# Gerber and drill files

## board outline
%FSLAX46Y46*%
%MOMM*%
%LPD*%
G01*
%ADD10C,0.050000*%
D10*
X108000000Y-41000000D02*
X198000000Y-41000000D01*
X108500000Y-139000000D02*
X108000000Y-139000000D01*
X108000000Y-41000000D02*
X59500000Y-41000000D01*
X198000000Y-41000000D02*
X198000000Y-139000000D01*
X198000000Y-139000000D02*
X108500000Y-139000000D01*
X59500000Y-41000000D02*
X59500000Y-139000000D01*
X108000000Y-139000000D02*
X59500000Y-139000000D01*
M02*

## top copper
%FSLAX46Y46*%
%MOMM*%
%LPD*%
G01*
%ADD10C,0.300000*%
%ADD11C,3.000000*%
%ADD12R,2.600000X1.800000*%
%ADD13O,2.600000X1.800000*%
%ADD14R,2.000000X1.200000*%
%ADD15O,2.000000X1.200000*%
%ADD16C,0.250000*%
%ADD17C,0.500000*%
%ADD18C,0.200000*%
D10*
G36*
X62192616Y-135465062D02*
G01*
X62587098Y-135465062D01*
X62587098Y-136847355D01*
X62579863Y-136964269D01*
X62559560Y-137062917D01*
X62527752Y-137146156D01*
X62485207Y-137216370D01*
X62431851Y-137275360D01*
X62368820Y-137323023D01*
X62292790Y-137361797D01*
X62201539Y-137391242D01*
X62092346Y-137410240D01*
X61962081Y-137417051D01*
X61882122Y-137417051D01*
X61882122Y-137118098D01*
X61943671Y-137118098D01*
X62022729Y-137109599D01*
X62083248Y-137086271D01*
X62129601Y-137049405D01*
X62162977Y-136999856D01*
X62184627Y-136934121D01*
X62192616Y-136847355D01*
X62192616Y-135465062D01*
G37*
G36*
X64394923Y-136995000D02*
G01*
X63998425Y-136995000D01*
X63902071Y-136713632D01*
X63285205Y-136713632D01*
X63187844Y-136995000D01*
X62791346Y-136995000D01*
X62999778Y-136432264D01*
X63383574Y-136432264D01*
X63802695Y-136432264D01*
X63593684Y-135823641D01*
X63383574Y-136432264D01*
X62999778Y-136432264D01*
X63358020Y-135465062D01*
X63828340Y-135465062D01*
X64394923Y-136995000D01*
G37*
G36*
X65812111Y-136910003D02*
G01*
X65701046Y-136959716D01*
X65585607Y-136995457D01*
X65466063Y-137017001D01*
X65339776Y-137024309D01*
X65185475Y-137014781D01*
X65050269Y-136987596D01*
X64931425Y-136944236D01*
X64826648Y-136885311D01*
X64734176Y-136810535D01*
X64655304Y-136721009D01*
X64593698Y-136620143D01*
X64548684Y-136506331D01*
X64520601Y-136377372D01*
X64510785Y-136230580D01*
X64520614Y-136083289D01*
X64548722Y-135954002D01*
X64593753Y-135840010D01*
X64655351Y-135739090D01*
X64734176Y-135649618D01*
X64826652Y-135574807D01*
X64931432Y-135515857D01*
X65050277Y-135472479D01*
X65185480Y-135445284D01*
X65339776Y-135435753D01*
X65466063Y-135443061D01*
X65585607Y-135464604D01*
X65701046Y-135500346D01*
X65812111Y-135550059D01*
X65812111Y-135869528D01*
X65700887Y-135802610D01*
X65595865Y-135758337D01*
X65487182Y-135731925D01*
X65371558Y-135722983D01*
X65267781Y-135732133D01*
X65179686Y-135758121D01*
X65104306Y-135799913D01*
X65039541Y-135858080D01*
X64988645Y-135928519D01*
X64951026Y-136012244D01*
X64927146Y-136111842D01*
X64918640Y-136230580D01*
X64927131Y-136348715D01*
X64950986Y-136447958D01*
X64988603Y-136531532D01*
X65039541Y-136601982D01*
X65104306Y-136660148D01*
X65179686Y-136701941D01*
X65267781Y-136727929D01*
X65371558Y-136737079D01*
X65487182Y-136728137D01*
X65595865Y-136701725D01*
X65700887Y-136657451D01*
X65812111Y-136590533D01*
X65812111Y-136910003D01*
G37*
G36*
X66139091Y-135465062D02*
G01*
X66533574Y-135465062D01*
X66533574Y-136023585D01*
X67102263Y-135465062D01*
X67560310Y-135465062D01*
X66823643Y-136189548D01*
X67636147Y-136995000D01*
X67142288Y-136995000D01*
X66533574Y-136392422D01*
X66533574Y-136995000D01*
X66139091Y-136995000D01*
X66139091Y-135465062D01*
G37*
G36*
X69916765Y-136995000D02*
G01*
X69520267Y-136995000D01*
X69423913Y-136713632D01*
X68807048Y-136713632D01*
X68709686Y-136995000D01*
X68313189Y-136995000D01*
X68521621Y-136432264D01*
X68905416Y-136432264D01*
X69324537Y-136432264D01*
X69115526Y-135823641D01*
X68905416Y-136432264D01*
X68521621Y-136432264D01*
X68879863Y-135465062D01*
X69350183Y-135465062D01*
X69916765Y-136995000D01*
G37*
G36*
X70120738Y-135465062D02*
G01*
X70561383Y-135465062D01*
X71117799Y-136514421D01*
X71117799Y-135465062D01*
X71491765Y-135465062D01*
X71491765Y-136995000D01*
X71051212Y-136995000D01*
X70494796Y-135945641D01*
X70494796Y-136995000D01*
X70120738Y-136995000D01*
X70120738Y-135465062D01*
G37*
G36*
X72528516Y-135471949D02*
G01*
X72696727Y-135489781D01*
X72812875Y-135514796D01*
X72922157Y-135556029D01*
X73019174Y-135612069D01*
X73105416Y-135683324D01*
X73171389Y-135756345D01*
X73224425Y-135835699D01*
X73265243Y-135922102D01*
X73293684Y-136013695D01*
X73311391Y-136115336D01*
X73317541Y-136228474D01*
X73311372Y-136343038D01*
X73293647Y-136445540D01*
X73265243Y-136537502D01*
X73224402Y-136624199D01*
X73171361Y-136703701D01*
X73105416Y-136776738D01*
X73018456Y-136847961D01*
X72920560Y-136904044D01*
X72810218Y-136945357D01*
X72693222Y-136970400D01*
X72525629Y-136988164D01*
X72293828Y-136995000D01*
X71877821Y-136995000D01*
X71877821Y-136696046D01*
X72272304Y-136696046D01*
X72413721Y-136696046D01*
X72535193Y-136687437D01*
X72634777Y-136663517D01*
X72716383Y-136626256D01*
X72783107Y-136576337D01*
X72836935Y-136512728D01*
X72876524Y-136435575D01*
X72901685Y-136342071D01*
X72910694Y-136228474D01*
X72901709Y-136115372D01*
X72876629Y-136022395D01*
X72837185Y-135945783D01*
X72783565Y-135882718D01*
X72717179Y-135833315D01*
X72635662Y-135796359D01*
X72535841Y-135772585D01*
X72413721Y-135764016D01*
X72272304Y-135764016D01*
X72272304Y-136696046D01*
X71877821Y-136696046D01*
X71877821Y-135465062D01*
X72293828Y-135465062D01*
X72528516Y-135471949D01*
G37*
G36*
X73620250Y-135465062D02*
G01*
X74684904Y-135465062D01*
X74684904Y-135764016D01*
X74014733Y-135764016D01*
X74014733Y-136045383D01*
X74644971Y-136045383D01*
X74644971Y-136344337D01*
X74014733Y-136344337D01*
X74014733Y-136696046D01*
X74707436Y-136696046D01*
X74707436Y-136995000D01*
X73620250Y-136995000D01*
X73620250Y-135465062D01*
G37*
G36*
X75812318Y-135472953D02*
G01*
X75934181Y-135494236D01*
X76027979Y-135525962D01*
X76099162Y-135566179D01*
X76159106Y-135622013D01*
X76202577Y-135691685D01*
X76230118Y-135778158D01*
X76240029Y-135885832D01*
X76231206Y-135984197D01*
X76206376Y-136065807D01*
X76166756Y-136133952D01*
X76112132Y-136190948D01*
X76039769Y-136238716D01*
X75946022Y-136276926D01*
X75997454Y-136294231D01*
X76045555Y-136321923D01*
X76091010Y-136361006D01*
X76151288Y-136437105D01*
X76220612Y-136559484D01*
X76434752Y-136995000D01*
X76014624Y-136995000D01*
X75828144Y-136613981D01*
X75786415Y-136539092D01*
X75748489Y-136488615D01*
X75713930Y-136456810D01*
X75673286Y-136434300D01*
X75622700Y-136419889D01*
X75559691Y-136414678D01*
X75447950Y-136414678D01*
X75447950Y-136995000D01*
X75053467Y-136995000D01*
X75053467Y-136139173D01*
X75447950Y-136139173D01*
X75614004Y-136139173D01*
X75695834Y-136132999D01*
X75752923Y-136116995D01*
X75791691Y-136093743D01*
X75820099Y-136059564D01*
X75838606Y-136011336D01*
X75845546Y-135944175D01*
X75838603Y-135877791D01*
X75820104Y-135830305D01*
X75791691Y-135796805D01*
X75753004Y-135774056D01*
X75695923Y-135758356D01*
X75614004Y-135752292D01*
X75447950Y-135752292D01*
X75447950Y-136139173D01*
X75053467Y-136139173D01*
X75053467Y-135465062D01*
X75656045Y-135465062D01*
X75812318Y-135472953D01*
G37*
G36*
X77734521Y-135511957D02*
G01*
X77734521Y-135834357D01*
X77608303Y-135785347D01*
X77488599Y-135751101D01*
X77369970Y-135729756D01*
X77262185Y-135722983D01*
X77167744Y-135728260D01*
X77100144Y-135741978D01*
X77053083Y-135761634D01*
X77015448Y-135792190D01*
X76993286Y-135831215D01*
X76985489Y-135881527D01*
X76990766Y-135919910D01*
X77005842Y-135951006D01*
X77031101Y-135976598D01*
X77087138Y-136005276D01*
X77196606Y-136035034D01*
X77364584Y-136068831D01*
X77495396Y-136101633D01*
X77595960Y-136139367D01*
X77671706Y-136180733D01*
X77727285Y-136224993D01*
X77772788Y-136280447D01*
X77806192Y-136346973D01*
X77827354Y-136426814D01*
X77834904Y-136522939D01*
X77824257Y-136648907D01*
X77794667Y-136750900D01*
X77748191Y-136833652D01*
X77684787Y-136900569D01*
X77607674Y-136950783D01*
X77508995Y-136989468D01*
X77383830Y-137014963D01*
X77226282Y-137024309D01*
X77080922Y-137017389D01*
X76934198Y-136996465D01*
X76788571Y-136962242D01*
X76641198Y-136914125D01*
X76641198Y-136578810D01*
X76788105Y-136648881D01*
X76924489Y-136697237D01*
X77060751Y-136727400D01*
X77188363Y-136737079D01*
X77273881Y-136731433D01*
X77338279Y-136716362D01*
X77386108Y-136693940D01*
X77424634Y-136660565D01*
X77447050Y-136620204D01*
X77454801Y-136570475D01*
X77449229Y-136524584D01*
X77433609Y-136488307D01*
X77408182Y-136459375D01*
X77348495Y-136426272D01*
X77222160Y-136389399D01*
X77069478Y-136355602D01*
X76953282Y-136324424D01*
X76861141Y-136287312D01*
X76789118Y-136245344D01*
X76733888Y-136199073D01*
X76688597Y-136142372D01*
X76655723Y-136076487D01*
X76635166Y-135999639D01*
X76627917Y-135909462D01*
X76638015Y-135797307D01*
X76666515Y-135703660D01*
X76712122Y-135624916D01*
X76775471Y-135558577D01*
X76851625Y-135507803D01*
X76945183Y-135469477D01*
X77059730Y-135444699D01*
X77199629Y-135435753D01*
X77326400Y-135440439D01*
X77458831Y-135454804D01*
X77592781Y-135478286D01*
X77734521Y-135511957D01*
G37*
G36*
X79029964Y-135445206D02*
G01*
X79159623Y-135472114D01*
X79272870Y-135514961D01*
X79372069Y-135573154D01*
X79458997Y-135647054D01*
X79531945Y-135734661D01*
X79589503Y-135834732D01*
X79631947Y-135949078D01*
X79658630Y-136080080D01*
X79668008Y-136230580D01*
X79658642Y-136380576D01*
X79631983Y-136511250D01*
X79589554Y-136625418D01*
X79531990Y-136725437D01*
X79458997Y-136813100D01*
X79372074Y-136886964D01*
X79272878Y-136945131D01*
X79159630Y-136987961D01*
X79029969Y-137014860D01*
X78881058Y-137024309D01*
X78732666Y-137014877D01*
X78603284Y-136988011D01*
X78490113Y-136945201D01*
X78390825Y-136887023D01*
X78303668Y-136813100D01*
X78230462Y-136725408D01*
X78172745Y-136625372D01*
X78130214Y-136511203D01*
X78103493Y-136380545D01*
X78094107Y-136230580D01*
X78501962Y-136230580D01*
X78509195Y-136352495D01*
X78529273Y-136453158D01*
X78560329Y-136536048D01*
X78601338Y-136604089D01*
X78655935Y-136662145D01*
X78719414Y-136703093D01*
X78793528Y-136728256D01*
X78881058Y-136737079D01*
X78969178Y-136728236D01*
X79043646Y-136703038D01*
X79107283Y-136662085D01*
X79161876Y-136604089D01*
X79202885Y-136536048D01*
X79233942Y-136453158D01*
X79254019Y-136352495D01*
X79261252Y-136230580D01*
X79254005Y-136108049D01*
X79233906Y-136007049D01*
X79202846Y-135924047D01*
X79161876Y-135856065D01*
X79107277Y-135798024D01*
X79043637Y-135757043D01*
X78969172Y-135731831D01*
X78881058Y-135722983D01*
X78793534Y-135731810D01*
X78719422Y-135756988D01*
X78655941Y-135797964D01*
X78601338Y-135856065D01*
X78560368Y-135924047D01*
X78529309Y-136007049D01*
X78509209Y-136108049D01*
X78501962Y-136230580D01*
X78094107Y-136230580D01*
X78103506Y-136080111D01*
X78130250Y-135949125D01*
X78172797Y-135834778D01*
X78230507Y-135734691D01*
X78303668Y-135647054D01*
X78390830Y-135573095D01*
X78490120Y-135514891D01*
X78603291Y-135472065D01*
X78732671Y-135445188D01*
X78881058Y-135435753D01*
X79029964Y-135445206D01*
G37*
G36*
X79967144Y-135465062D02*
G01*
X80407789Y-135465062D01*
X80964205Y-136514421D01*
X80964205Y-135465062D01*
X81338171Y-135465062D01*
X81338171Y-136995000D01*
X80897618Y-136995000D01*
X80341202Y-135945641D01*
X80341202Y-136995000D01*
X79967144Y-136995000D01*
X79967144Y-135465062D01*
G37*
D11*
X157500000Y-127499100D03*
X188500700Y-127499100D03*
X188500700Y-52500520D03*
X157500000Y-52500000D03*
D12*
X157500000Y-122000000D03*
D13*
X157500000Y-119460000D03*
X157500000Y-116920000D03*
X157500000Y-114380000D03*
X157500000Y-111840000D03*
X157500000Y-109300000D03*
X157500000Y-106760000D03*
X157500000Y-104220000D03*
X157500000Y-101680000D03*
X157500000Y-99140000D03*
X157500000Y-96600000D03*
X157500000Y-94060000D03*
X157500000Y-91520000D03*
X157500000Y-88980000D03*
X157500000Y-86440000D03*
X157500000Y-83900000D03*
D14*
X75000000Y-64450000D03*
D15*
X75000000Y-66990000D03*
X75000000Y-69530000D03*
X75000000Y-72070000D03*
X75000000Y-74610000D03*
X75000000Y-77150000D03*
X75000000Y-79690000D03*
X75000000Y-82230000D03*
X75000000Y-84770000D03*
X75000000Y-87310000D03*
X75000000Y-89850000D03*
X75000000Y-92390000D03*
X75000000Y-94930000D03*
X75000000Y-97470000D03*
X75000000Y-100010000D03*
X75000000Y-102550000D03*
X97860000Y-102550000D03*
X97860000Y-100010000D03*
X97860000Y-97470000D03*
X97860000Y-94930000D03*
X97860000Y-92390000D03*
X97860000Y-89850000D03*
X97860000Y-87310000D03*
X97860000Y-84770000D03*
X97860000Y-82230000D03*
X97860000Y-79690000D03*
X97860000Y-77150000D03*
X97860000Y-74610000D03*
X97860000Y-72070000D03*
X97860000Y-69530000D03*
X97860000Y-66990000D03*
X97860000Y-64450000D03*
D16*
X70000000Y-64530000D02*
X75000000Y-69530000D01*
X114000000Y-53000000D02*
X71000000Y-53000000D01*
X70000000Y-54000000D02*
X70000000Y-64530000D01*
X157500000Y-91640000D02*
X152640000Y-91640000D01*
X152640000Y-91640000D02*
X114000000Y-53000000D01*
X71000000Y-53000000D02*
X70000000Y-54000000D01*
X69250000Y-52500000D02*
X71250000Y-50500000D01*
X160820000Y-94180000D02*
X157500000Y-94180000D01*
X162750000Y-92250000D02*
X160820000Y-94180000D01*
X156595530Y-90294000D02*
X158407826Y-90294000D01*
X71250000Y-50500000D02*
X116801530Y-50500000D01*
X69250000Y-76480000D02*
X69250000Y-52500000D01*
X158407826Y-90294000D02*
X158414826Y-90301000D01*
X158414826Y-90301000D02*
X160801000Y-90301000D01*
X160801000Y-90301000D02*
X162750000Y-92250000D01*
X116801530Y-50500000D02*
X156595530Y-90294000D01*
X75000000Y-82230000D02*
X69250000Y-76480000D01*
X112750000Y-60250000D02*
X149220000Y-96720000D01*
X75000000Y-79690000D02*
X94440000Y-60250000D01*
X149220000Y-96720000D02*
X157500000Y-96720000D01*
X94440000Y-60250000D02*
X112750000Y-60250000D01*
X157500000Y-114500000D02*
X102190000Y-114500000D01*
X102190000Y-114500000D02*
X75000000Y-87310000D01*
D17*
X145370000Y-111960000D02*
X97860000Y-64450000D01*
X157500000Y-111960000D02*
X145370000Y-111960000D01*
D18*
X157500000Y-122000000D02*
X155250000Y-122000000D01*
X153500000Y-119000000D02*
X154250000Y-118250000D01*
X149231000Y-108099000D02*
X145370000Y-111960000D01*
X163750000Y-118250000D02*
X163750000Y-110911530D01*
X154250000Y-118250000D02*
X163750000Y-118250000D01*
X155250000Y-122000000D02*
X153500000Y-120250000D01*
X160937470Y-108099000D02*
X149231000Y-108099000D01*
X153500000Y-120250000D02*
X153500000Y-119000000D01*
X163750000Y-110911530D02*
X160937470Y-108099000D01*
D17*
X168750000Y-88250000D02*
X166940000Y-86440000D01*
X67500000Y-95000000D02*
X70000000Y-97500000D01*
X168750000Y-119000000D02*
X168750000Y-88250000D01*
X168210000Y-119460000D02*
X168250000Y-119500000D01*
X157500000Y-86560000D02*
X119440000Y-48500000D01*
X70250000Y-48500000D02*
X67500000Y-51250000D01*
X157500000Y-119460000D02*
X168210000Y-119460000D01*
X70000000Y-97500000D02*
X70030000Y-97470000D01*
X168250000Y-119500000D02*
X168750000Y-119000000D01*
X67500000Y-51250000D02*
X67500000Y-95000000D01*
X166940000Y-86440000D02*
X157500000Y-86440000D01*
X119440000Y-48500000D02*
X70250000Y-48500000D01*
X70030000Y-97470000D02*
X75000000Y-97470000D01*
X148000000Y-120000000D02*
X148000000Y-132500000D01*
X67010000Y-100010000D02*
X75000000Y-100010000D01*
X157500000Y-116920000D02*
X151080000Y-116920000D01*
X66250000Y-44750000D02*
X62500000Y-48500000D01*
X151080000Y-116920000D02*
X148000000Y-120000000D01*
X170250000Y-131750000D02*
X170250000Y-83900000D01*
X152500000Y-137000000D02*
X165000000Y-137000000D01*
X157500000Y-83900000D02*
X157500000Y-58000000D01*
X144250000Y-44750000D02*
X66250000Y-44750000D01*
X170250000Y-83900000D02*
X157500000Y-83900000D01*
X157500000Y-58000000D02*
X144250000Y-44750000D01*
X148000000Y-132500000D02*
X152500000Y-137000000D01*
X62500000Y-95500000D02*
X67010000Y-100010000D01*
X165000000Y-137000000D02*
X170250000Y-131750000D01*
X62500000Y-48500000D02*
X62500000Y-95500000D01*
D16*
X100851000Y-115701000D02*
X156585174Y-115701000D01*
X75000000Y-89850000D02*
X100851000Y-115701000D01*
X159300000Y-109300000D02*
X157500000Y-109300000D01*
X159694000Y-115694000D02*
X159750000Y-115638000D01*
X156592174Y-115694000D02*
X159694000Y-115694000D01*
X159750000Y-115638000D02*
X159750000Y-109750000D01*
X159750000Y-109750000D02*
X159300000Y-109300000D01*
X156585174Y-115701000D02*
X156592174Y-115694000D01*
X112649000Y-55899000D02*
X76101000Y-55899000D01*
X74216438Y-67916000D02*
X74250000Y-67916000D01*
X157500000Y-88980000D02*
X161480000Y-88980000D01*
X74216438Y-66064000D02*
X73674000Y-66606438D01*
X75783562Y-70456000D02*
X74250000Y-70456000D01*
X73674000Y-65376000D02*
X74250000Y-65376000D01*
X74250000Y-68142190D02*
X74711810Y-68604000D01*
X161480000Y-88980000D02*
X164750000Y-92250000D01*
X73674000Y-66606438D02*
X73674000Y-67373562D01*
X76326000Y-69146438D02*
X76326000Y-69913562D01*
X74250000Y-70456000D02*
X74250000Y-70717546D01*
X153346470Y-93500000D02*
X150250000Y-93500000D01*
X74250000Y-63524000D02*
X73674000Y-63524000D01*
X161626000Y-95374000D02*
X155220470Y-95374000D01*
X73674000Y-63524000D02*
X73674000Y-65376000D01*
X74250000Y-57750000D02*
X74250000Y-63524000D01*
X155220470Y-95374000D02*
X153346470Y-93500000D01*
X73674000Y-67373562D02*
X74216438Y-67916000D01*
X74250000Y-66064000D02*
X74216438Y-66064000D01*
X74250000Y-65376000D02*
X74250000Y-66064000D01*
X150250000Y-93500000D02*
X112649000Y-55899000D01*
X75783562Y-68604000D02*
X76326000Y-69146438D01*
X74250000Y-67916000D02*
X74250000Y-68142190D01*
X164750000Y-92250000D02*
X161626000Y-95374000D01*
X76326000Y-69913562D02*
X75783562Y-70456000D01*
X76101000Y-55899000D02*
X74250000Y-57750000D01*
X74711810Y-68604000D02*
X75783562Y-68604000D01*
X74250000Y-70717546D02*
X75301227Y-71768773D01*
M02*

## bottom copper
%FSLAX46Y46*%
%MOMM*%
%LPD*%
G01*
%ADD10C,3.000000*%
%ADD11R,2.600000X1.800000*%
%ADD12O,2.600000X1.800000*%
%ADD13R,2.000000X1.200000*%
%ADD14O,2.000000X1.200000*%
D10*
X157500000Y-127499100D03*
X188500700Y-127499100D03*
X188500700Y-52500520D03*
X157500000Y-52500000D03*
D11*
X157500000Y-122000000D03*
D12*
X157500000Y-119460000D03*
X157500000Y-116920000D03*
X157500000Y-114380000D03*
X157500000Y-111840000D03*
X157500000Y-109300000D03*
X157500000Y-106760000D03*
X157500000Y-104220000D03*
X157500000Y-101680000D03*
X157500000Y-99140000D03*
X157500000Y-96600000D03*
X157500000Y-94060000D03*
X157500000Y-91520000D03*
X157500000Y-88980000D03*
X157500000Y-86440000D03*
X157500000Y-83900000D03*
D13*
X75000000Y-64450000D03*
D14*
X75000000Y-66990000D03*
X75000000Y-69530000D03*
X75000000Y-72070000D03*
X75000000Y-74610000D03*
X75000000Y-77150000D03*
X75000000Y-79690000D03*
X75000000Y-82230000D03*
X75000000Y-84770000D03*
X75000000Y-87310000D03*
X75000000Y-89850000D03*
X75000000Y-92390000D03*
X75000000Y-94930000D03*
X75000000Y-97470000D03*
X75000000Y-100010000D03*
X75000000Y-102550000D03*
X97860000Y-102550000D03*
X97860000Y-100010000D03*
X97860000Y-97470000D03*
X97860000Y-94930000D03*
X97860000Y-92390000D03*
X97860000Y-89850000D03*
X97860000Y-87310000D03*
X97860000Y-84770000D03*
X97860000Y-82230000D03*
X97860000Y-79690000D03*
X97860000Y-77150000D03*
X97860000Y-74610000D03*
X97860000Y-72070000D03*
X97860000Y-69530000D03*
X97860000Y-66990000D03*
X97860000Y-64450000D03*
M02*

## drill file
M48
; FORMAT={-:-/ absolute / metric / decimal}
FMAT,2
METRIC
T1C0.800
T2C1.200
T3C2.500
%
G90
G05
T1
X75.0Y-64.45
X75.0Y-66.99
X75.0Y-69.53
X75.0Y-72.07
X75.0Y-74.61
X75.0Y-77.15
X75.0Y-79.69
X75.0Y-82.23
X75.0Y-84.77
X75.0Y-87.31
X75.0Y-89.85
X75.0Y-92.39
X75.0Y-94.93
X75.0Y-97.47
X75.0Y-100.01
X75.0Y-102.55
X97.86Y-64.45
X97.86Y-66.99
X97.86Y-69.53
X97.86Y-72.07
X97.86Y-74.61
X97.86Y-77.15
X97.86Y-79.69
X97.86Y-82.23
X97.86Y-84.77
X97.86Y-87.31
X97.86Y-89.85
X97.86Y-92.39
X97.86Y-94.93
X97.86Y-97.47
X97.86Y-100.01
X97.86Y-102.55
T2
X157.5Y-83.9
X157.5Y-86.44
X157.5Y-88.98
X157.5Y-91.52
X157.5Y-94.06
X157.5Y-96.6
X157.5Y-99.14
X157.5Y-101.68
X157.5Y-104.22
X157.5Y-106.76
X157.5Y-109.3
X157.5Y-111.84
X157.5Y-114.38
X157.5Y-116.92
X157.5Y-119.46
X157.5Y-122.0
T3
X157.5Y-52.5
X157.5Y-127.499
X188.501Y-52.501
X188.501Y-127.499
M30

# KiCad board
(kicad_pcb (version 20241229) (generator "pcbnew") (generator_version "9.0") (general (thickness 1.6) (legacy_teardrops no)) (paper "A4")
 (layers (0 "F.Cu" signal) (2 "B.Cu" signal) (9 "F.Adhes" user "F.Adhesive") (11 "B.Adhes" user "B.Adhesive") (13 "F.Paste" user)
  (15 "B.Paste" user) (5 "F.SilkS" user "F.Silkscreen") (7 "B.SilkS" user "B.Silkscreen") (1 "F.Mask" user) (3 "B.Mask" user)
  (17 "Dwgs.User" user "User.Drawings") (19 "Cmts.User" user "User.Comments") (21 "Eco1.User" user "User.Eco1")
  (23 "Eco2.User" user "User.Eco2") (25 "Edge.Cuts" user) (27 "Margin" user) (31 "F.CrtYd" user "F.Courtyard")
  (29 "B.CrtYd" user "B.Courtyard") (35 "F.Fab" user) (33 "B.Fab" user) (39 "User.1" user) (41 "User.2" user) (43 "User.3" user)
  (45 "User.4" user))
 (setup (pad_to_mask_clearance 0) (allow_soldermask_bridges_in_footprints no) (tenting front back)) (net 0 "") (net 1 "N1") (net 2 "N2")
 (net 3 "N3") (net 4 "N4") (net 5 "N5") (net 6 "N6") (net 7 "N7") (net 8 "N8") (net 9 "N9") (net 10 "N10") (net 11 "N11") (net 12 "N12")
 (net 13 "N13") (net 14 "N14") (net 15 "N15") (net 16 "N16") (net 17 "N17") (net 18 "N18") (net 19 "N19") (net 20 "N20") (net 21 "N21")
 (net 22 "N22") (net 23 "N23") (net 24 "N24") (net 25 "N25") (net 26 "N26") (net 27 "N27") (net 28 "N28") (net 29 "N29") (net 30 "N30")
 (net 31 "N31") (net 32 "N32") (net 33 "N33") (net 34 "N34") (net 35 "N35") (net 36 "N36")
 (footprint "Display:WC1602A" (layer "F.Cu") (at 157.5 122 90)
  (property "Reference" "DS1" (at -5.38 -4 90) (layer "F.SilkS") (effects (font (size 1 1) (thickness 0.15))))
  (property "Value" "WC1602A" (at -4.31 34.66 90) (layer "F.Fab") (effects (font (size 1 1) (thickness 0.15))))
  (pad "" thru_hole circle (at -5.4991 0 90) (size 3 3) (drill 2.5) (layers "*.Cu" "*.Mask") (remove_unused_layers no))
  (pad "" thru_hole circle (at -5.4991 31.0007 90) (size 3 3) (drill 2.5) (layers "*.Cu" "*.Mask") (remove_unused_layers no))
  (pad "" thru_hole circle (at 69.49948 31.0007 90) (size 3 3) (drill 2.5) (layers "*.Cu" "*.Mask") (remove_unused_layers no))
  (pad "" thru_hole circle (at 69.5 0 90) (size 3 3) (drill 2.5) (layers "*.Cu" "*.Mask") (remove_unused_layers no))
  (pad "1" thru_hole rect (at 0 0 90) (size 1.8 2.6) (drill 1.2) (layers "*.Cu" "*.Mask") (remove_unused_layers no) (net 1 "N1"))
  (pad "2" thru_hole oval (at 2.54 0 90) (size 1.8 2.6) (drill 1.2) (layers "*.Cu" "*.Mask") (remove_unused_layers no) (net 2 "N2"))
  (pad "3" thru_hole oval (at 5.08 0 90) (size 1.8 2.6) (drill 1.2) (layers "*.Cu" "*.Mask") (remove_unused_layers no) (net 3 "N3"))
  (pad "4" thru_hole oval (at 7.62 0 90) (size 1.8 2.6) (drill 1.2) (layers "*.Cu" "*.Mask") (remove_unused_layers no) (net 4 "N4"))
  (pad "5" thru_hole oval (at 10.16 0 90) (size 1.8 2.6) (drill 1.2) (layers "*.Cu" "*.Mask") (remove_unused_layers no) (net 1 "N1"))
  (pad "6" thru_hole oval (at 12.7 0 90) (size 1.8 2.6) (drill 1.2) (layers "*.Cu" "*.Mask") (remove_unused_layers no) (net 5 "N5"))
  (pad "7" thru_hole oval (at 15.24 0 90) (size 1.8 2.6) (drill 1.2) (layers "*.Cu" "*.Mask") (remove_unused_layers no) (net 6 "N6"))
  (pad "8" thru_hole oval (at 17.78 0 90) (size 1.8 2.6) (drill 1.2) (layers "*.Cu" "*.Mask") (remove_unused_layers no) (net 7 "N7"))
  (pad "9" thru_hole oval (at 20.32 0 90) (size 1.8 2.6) (drill 1.2) (layers "*.Cu" "*.Mask") (remove_unused_layers no) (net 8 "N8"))
  (pad "10" thru_hole oval (at 22.86 0 90) (size 1.8 2.6) (drill 1.2) (layers "*.Cu" "*.Mask") (remove_unused_layers no) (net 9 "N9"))
  (pad "11" thru_hole oval (at 25.4 0 90) (size 1.8 2.6) (drill 1.2) (layers "*.Cu" "*.Mask") (remove_unused_layers no) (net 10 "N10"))
  (pad "12" thru_hole oval (at 27.94 0 90) (size 1.8 2.6) (drill 1.2) (layers "*.Cu" "*.Mask") (remove_unused_layers no) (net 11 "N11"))
  (pad "13" thru_hole oval (at 30.48 0 90) (size 1.8 2.6) (drill 1.2) (layers "*.Cu" "*.Mask") (remove_unused_layers no) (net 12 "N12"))
  (pad "14" thru_hole oval (at 33.02 0 90) (size 1.8 2.6) (drill 1.2) (layers "*.Cu" "*.Mask") (remove_unused_layers no) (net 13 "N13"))
  (pad "15" thru_hole oval (at 35.56 0 90) (size 1.8 2.6) (drill 1.2) (layers "*.Cu" "*.Mask") (remove_unused_layers no) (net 2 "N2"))
  (pad "16" thru_hole oval (at 38.1 0 90) (size 1.8 2.6) (drill 1.2) (layers "*.Cu" "*.Mask") (remove_unused_layers no) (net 3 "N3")))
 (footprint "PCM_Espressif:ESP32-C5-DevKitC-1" (layer "F.Cu") (at 74.96012 64.45468)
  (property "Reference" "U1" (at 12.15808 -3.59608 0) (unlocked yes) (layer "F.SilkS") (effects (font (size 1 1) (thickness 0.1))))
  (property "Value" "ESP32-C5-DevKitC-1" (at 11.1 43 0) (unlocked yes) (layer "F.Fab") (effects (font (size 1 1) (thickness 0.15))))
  (pad "1" thru_hole rect (at 0.03988 -0.00468 270) (size 1.2 2) (drill 0.8) (layers "*.Cu" "*.Mask") (remove_unused_layers no)
   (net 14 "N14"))
  (pad "2" thru_hole oval (at 0.03988 2.53532 270) (size 1.2 2) (drill 0.8) (layers "*.Cu" "*.Mask") (remove_unused_layers no)
   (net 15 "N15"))
  (pad "3" thru_hole oval (at 0.03988 5.07532 270) (size 1.2 2) (drill 0.8) (layers "*.Cu" "*.Mask") (remove_unused_layers no)
   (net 12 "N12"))
  (pad "4" thru_hole oval (at 0.03988 7.61532 270) (size 1.2 2) (drill 0.8) (layers "*.Cu" "*.Mask") (remove_unused_layers no)
   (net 13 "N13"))
  (pad "5" thru_hole oval (at 0.03988 10.15532 270) (size 1.2 2) (drill 0.8) (layers "*.Cu" "*.Mask") (remove_unused_layers no)
   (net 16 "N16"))
  (pad "6" thru_hole oval (at 0.03988 12.69532 270) (size 1.2 2) (drill 0.8) (layers "*.Cu" "*.Mask") (remove_unused_layers no)
   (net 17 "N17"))
  (pad "7" thru_hole oval (at 0.03988 15.23532 270) (size 1.2 2) (drill 0.8) (layers "*.Cu" "*.Mask") (remove_unused_layers no)
   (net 10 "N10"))
  (pad "8" thru_hole oval (at 0.03988 17.77532 270) (size 1.2 2) (drill 0.8) (layers "*.Cu" "*.Mask") (remove_unused_layers no)
   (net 11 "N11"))
  (pad "9" thru_hole oval (at 0.03988 20.31532 270) (size 1.2 2) (drill 0.8) (layers "*.Cu" "*.Mask") (remove_unused_layers no)
   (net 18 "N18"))
  (pad "10" thru_hole oval (at 0.03988 22.85532 270) (size 1.2 2) (drill 0.8) (layers "*.Cu" "*.Mask") (remove_unused_layers no)
   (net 4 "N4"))
  (pad "11" thru_hole oval (at 0.03988 25.39532 270) (size 1.2 2) (drill 0.8) (layers "*.Cu" "*.Mask") (remove_unused_layers no)
   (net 5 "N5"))
  (pad "12" thru_hole oval (at 0.03988 27.93532 270) (size 1.2 2) (drill 0.8) (layers "*.Cu" "*.Mask") (remove_unused_layers no)
   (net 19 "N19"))
  (pad "13" thru_hole oval (at 0.03988 30.47532 270) (size 1.2 2) (drill 0.8) (layers "*.Cu" "*.Mask") (remove_unused_layers no)
   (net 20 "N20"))
  (pad "14" thru_hole oval (at 0.03988 33.01532 270) (size 1.2 2) (drill 0.8) (layers "*.Cu" "*.Mask") (remove_unused_layers no)
   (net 2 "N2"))
  (pad "15" thru_hole oval (at 0.03988 35.55532 270) (size 1.2 2) (drill 0.8) (layers "*.Cu" "*.Mask") (remove_unused_layers no)
   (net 3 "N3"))
  (pad "16" thru_hole oval (at 0.03988 38.09532 270) (size 1.2 2) (drill 0.8) (layers "*.Cu" "*.Mask") (remove_unused_layers no)
   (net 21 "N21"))
  (pad "17" thru_hole oval (at 22.89988 38.09532 270) (size 1.2 2) (drill 0.8) (layers "*.Cu" "*.Mask") (remove_unused_layers no)
   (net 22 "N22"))
  (pad "18" thru_hole oval (at 22.89988 35.55532 270) (size 1.2 2) (drill 0.8) (layers "*.Cu" "*.Mask") (remove_unused_layers no)
   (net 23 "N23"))
  (pad "19" thru_hole oval (at 22.89988 33.01532 270) (size 1.2 2) (drill 0.8) (layers "*.Cu" "*.Mask") (remove_unused_layers no)
   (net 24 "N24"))
  (pad "20" thru_hole oval (at 22.89988 30.47532 270) (size 1.2 2) (drill 0.8) (layers "*.Cu" "*.Mask") (remove_unused_layers no)
   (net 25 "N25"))
  (pad "21" thru_hole oval (at 22.89988 27.93532 270) (size 1.2 2) (drill 0.8) (layers "*.Cu" "*.Mask") (remove_unused_layers no)
   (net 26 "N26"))
  (pad "22" thru_hole oval (at 22.89988 25.39532 270) (size 1.2 2) (drill 0.8) (layers "*.Cu" "*.Mask") (remove_unused_layers no)
   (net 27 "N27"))
  (pad "23" thru_hole oval (at 22.89988 22.85532 270) (size 1.2 2) (drill 0.8) (layers "*.Cu" "*.Mask") (remove_unused_layers no)
   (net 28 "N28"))
  (pad "24" thru_hole oval (at 22.89988 20.31532 270) (size 1.2 2) (drill 0.8) (layers "*.Cu" "*.Mask") (remove_unused_layers no)
   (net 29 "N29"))
  (pad "25" thru_hole oval (at 22.89988 17.77532 270) (size 1.2 2) (drill 0.8) (layers "*.Cu" "*.Mask") (remove_unused_layers no)
   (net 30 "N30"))
  (pad "26" thru_hole oval (at 22.89988 15.23532 270) (size 1.2 2) (drill 0.8) (layers "*.Cu" "*.Mask") (remove_unused_layers no)
   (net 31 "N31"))
  (pad "27" thru_hole oval (at 22.89988 12.69532 270) (size 1.2 2) (drill 0.8) (layers "*.Cu" "*.Mask") (remove_unused_layers no)
   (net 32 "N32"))
  (pad "28" thru_hole oval (at 22.89988 10.15532 270) (size 1.2 2) (drill 0.8) (layers "*.Cu" "*.Mask") (remove_unused_layers no)
   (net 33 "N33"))
  (pad "29" thru_hole oval (at 22.89988 7.61532 270) (size 1.2 2) (drill 0.8) (layers "*.Cu" "*.Mask") (remove_unused_layers no)
   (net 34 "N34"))
  (pad "30" thru_hole oval (at 22.89988 5.07532 270) (size 1.2 2) (drill 0.8) (layers "*.Cu" "*.Mask") (remove_unused_layers no)
   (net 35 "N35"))
  (pad "31" thru_hole oval (at 22.89988 2.53532 270) (size 1.2 2) (drill 0.8) (layers "*.Cu" "*.Mask") (remove_unused_layers no)
   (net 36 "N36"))
  (pad "32" thru_hole oval (at 22.89988 -0.00468 270) (size 1.2 2) (drill 0.8) (layers "*.Cu" "*.Mask") (remove_unused_layers no)
   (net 1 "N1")))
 (gr_line (start 108 41) (end 198 41) (stroke (width 0.05) (type default)) (layer "Edge.Cuts"))
 (gr_line (start 108.5 139) (end 108 139) (stroke (width 0.05) (type default)) (layer "Edge.Cuts"))
 (gr_line (start 108 41) (end 59.5 41) (stroke (width 0.05) (type default)) (layer "Edge.Cuts"))
 (gr_line (start 198 41) (end 198 139) (stroke (width 0.05) (type default)) (layer "Edge.Cuts"))
 (gr_line (start 198 139) (end 108.5 139) (stroke (width 0.05) (type default)) (layer "Edge.Cuts"))
 (gr_line (start 59.5 41) (end 59.5 139) (stroke (width 0.05) (type default)) (layer "Edge.Cuts"))
 (gr_line (start 108 139) (end 59.5 139) (stroke (width 0.05) (type default)) (layer "Edge.Cuts"))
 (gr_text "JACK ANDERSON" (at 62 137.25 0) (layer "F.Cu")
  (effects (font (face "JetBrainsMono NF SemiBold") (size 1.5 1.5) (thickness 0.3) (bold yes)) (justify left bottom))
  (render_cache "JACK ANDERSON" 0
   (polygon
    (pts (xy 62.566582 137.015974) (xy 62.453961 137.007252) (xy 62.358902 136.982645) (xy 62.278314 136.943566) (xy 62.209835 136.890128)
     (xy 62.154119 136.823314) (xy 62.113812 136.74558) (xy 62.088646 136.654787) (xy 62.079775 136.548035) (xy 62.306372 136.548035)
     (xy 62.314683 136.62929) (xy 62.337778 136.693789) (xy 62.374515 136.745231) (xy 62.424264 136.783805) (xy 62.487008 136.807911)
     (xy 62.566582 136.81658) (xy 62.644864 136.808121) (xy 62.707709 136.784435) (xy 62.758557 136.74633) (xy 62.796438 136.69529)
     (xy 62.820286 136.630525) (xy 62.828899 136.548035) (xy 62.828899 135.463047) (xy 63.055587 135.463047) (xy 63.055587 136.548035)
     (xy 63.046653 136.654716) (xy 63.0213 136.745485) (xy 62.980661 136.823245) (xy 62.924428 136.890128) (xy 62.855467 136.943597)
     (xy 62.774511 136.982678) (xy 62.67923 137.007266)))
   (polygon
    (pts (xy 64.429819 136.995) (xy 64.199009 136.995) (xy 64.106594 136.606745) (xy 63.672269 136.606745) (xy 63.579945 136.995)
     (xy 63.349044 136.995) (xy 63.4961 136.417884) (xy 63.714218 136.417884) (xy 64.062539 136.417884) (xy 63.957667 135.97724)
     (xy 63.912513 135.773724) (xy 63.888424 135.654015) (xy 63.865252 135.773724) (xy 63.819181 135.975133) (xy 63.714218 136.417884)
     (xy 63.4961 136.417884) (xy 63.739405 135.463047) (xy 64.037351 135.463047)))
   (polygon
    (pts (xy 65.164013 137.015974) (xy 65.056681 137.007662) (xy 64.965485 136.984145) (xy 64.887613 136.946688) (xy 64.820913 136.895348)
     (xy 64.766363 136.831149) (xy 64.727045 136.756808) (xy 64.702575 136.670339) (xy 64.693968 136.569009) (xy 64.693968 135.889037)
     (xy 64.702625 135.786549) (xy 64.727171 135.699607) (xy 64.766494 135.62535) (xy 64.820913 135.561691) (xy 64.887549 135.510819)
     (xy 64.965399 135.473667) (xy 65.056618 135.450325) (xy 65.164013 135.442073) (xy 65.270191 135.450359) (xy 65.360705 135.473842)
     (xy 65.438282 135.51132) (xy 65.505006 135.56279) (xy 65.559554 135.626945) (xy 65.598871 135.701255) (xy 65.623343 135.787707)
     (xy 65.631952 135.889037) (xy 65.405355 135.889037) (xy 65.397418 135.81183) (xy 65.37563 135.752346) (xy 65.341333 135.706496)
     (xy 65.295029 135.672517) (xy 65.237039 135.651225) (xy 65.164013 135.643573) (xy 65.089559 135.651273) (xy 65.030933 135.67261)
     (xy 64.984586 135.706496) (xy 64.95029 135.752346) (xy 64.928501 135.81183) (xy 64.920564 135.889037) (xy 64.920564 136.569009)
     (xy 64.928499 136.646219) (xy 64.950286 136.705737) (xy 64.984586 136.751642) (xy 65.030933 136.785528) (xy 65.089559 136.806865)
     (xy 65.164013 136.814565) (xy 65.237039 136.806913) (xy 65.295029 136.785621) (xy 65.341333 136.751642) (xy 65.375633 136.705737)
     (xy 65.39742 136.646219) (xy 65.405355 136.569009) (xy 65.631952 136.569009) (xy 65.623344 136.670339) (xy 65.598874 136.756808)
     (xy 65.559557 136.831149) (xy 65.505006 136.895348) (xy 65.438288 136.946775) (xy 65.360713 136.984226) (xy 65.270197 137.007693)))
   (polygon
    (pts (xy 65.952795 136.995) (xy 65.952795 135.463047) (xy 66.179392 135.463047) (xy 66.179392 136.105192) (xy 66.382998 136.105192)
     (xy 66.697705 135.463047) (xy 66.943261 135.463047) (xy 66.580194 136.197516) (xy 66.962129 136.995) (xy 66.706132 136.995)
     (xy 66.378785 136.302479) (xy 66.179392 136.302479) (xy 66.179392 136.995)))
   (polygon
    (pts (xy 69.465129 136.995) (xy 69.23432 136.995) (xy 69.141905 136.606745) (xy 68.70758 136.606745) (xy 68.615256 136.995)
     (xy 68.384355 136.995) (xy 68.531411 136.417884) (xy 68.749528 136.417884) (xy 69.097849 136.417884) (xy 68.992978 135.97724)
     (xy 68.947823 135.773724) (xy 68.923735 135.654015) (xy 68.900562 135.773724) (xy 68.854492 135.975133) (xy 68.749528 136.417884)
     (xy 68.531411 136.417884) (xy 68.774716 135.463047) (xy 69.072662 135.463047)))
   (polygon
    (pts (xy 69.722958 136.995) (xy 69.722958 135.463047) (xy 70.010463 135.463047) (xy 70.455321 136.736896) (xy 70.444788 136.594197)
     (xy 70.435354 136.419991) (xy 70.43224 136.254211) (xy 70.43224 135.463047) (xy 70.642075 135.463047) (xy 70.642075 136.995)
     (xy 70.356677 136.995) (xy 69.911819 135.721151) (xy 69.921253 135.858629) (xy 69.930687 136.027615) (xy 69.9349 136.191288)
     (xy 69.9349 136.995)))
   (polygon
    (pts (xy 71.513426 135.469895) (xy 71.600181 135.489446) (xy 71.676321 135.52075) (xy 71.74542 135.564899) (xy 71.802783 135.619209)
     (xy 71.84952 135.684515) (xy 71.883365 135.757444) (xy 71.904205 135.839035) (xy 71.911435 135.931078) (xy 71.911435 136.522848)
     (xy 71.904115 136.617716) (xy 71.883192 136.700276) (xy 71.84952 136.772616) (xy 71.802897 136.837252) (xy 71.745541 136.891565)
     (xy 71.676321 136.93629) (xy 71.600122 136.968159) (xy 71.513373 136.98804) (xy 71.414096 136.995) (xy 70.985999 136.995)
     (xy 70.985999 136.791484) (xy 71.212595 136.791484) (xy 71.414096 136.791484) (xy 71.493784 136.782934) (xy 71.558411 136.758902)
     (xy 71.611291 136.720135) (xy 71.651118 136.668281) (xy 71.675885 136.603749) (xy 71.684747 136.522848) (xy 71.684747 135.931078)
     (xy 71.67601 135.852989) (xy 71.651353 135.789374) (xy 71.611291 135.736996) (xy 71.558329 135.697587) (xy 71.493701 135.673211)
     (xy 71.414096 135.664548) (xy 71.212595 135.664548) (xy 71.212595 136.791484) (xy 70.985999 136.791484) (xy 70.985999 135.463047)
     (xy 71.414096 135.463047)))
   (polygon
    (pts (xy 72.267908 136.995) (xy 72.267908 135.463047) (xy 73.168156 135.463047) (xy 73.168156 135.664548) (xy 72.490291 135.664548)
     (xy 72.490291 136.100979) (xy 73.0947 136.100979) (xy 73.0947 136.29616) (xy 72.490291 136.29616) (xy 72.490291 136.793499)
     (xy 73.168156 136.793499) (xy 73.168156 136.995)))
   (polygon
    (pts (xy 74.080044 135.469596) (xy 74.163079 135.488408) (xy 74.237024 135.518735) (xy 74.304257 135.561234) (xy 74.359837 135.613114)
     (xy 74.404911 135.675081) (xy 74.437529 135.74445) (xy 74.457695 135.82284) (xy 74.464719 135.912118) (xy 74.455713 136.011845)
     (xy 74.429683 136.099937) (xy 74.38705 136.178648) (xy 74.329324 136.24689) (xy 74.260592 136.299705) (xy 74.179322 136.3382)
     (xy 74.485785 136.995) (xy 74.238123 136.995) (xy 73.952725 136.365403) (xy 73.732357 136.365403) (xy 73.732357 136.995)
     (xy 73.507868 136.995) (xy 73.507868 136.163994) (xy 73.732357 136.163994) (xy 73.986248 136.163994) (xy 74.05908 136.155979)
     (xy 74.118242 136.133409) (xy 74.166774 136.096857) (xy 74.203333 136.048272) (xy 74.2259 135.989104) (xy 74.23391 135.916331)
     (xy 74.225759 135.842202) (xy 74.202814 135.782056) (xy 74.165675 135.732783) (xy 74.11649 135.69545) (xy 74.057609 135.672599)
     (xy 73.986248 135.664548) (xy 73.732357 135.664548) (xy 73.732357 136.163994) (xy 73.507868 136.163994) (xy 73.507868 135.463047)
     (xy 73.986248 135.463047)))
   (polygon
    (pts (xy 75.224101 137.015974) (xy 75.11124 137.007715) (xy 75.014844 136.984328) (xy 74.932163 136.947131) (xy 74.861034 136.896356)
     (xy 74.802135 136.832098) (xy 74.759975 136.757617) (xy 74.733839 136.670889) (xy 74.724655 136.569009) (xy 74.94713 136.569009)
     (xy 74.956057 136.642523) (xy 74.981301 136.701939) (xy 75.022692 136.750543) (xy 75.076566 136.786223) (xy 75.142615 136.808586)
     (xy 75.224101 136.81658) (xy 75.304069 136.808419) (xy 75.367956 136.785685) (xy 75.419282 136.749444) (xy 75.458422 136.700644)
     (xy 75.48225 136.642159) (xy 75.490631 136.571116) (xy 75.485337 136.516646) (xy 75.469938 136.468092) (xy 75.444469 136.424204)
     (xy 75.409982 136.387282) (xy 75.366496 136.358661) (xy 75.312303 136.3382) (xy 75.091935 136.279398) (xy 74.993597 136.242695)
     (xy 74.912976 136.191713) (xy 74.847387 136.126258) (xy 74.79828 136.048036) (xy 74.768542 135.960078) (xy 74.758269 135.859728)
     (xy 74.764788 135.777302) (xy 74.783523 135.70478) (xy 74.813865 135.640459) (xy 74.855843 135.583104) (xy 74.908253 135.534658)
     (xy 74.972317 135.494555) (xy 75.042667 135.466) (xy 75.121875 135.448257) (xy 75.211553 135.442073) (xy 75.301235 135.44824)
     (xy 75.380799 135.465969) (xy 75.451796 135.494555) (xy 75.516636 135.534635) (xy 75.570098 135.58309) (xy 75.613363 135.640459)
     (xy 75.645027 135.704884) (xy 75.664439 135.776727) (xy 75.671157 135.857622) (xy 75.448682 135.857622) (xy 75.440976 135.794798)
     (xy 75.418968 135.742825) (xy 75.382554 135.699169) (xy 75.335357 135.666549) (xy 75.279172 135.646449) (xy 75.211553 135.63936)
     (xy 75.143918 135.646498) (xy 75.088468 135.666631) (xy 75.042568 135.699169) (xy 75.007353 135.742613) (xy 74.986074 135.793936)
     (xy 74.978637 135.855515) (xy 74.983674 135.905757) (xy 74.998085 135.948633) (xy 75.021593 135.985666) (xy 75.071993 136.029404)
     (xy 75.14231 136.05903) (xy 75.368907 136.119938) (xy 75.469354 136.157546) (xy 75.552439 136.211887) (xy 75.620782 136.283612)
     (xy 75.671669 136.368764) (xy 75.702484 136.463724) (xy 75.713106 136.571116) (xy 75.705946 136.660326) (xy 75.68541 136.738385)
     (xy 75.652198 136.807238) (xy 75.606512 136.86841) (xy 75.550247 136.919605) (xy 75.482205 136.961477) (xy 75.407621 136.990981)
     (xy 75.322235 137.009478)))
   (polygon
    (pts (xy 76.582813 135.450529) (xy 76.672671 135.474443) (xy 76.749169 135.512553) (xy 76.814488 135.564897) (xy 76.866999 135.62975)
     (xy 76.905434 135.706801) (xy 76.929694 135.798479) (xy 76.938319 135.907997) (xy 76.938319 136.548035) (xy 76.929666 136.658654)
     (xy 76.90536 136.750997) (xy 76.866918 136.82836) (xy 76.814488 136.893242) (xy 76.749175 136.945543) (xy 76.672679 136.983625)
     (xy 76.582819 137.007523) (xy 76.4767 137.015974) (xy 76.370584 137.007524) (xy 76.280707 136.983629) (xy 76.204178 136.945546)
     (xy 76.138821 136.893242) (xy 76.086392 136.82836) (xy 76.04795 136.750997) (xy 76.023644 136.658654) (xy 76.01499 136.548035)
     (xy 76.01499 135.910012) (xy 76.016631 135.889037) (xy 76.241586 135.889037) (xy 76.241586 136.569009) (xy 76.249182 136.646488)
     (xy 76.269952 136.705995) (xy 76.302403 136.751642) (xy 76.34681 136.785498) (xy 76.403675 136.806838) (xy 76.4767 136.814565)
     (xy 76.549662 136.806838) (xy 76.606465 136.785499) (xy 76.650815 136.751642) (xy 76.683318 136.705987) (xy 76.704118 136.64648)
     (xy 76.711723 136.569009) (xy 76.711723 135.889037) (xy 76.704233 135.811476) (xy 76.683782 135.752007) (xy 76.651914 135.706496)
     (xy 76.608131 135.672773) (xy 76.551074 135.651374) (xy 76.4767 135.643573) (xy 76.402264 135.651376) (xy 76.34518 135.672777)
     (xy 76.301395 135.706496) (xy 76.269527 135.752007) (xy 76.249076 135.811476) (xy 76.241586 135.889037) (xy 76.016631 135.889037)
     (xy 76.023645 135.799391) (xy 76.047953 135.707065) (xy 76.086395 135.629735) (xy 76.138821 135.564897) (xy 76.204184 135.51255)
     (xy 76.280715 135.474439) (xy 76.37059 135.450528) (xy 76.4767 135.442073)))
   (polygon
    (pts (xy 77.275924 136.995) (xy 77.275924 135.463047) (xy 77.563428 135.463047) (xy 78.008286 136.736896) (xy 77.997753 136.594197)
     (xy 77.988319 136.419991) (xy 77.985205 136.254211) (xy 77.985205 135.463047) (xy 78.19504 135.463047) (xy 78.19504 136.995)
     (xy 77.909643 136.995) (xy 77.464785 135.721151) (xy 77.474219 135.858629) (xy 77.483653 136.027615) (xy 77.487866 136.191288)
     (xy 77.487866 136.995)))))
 (segment (start 70 64.53) (end 75 69.53) (width 0.25) (layer "F.Cu") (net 12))
 (segment (start 114 53) (end 71 53) (width 0.25) (layer "F.Cu") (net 12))
 (segment (start 70 54) (end 70 64.53) (width 0.25) (layer "F.Cu") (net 12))
 (segment (start 157.5 91.64) (end 152.64 91.64) (width 0.25) (layer "F.Cu") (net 12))
 (segment (start 152.64 91.64) (end 114 53) (width 0.25) (layer "F.Cu") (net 12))
 (segment (start 71 53) (end 70 54) (width 0.25) (layer "F.Cu") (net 12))
 (segment (start 69.25 52.5) (end 71.25 50.5) (width 0.25) (layer "F.Cu") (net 11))
 (segment (start 160.82 94.18) (end 157.5 94.18) (width 0.25) (layer "F.Cu") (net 11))
 (segment (start 162.75 92.25) (end 160.82 94.18) (width 0.25) (layer "F.Cu") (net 11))
 (segment (start 156.59553 90.294) (end 158.407826 90.294) (width 0.25) (layer "F.Cu") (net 11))
 (segment (start 71.25 50.5) (end 116.80153 50.5) (width 0.25) (layer "F.Cu") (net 11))
 (segment (start 69.25 76.48) (end 69.25 52.5) (width 0.25) (layer "F.Cu") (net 11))
 (segment (start 158.407826 90.294) (end 158.414826 90.301) (width 0.25) (layer "F.Cu") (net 11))
 (segment (start 158.414826 90.301) (end 160.801 90.301) (width 0.25) (layer "F.Cu") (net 11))
 (segment (start 160.801 90.301) (end 162.75 92.25) (width 0.25) (layer "F.Cu") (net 11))
 (segment (start 116.80153 50.5) (end 156.59553 90.294) (width 0.25) (layer "F.Cu") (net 11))
 (segment (start 75 82.23) (end 69.25 76.48) (width 0.25) (layer "F.Cu") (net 11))
 (segment (start 112.75 60.25) (end 149.22 96.72) (width 0.25) (layer "F.Cu") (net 10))
 (segment (start 75 79.69) (end 94.44 60.25) (width 0.25) (layer "F.Cu") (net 10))
 (segment (start 149.22 96.72) (end 157.5 96.72) (width 0.25) (layer "F.Cu") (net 10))
 (segment (start 94.44 60.25) (end 112.75 60.25) (width 0.25) (layer "F.Cu") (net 10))
 (segment (start 157.5 114.5) (end 102.19 114.5) (width 0.25) (layer "F.Cu") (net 4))
 (segment (start 102.19 114.5) (end 75 87.31) (width 0.25) (layer "F.Cu") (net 4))
 (segment (start 145.37 111.96) (end 97.86 64.45) (width 0.5) (layer "F.Cu") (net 1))
 (segment (start 157.5 111.96) (end 145.37 111.96) (width 0.5) (layer "F.Cu") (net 1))
 (segment (start 157.5 122) (end 155.25 122) (width 0.2) (layer "F.Cu") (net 1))
 (segment (start 153.5 119) (end 154.25 118.25) (width 0.2) (layer "F.Cu") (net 1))
 (segment (start 149.231 108.099) (end 145.37 111.96) (width 0.2) (layer "F.Cu") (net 1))
 (segment (start 163.75 118.25) (end 163.75 110.91153) (width 0.2) (layer "F.Cu") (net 1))
 (segment (start 154.25 118.25) (end 163.75 118.25) (width 0.2) (layer "F.Cu") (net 1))
 (segment (start 155.25 122) (end 153.5 120.25) (width 0.2) (layer "F.Cu") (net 1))
 (segment (start 160.93747 108.099) (end 149.231 108.099) (width 0.2) (layer "F.Cu") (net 1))
 (segment (start 153.5 120.25) (end 153.5 119) (width 0.2) (layer "F.Cu") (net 1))
 (segment (start 163.75 110.91153) (end 160.93747 108.099) (width 0.2) (layer "F.Cu") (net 1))
 (segment (start 168.75 88.25) (end 166.94 86.44) (width 0.5) (layer "F.Cu") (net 2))
 (segment (start 67.5 95) (end 70 97.5) (width 0.5) (layer "F.Cu") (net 2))
 (segment (start 168.75 119) (end 168.75 88.25) (width 0.5) (layer "F.Cu") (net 2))
 (segment (start 168.21 119.46) (end 168.25 119.5) (width 0.5) (layer "F.Cu") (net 2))
 (segment (start 157.5 86.56) (end 119.44 48.5) (width 0.5) (layer "F.Cu") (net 2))
 (segment (start 70.25 48.5) (end 67.5 51.25) (width 0.5) (layer "F.Cu") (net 2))
 (segment (start 157.5 119.46) (end 168.21 119.46) (width 0.5) (layer "F.Cu") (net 2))
 (segment (start 70 97.5) (end 70.03 97.47) (width 0.5) (layer "F.Cu") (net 2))
 (segment (start 168.25 119.5) (end 168.75 119) (width 0.5) (layer "F.Cu") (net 2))
 (segment (start 67.5 51.25) (end 67.5 95) (width 0.5) (layer "F.Cu") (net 2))
 (segment (start 166.94 86.44) (end 157.5 86.44) (width 0.5) (layer "F.Cu") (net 2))
 (segment (start 119.44 48.5) (end 70.25 48.5) (width 0.5) (layer "F.Cu") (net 2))
 (segment (start 70.03 97.47) (end 75 97.47) (width 0.5) (layer "F.Cu") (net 2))
 (segment (start 148 120) (end 148 132.5) (width 0.5) (layer "F.Cu") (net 3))
 (segment (start 67.01 100.01) (end 75 100.01) (width 0.5) (layer "F.Cu") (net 3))
 (segment (start 157.5 116.92) (end 151.08 116.92) (width 0.5) (layer "F.Cu") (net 3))
 (segment (start 66.25 44.75) (end 62.5 48.5) (width 0.5) (layer "F.Cu") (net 3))
 (segment (start 151.08 116.92) (end 148 120) (width 0.5) (layer "F.Cu") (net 3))
 (segment (start 170.25 131.75) (end 170.25 83.9) (width 0.5) (layer "F.Cu") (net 3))
 (segment (start 152.5 137) (end 165 137) (width 0.5) (layer "F.Cu") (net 3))
 (segment (start 157.5 83.9) (end 157.5 58) (width 0.5) (layer "F.Cu") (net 3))
 (segment (start 144.25 44.75) (end 66.25 44.75) (width 0.5) (layer "F.Cu") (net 3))
 (segment (start 170.25 83.9) (end 157.5 83.9) (width 0.5) (layer "F.Cu") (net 3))
 (segment (start 157.5 58) (end 144.25 44.75) (width 0.5) (layer "F.Cu") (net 3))
 (segment (start 148 132.5) (end 152.5 137) (width 0.5) (layer "F.Cu") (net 3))
 (segment (start 62.5 95.5) (end 67.01 100.01) (width 0.5) (layer "F.Cu") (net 3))
 (segment (start 165 137) (end 170.25 131.75) (width 0.5) (layer "F.Cu") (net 3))
 (segment (start 62.5 48.5) (end 62.5 95.5) (width 0.5) (layer "F.Cu") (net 3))
 (segment (start 100.851 115.701) (end 156.585174 115.701) (width 0.25) (layer "F.Cu") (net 5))
 (segment (start 75 89.85) (end 100.851 115.701) (width 0.25) (layer "F.Cu") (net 5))
 (segment (start 159.3 109.3) (end 157.5 109.3) (width 0.25) (layer "F.Cu") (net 5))
 (segment (start 159.694 115.694) (end 159.75 115.638) (width 0.25) (layer "F.Cu") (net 5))
 (segment (start 156.592174 115.694) (end 159.694 115.694) (width 0.25) (layer "F.Cu") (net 5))
 (segment (start 159.75 115.638) (end 159.75 109.75) (width 0.25) (layer "F.Cu") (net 5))
 (segment (start 159.75 109.75) (end 159.3 109.3) (width 0.25) (layer "F.Cu") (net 5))
 (segment (start 156.585174 115.701) (end 156.592174 115.694) (width 0.25) (layer "F.Cu") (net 5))
 (segment (start 112.649 55.899) (end 76.101 55.899) (width 0.25) (layer "F.Cu") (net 13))
 (segment (start 74.216438 67.916) (end 74.25 67.916) (width 0.25) (layer "F.Cu") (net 13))
 (segment (start 157.5 88.98) (end 161.48 88.98) (width 0.25) (layer "F.Cu") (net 13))
 (segment (start 74.216438 66.064) (end 73.674 66.606438) (width 0.25) (layer "F.Cu") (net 13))
 (segment (start 75.783562 70.456) (end 74.25 70.456) (width 0.25) (layer "F.Cu") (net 13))
 (segment (start 73.674 65.376) (end 74.25 65.376) (width 0.25) (layer "F.Cu") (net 13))
 (segment (start 74.25 68.14219) (end 74.71181 68.604) (width 0.25) (layer "F.Cu") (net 13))
 (segment (start 161.48 88.98) (end 164.75 92.25) (width 0.25) (layer "F.Cu") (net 13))
 (segment (start 73.674 66.606438) (end 73.674 67.373562) (width 0.25) (layer "F.Cu") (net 13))
 (segment (start 76.326 69.146438) (end 76.326 69.913562) (width 0.25) (layer "F.Cu") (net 13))
 (segment (start 74.25 70.456) (end 74.25 70.717546) (width 0.25) (layer "F.Cu") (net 13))
 (segment (start 153.34647 93.5) (end 150.25 93.5) (width 0.25) (layer "F.Cu") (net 13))
 (segment (start 74.25 63.524) (end 73.674 63.524) (width 0.25) (layer "F.Cu") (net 13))
 (segment (start 161.626 95.374) (end 155.22047 95.374) (width 0.25) (layer "F.Cu") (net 13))
 (segment (start 73.674 63.524) (end 73.674 65.376) (width 0.25) (layer "F.Cu") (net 13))
 (segment (start 74.25 57.75) (end 74.25 63.524) (width 0.25) (layer "F.Cu") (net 13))
 (segment (start 155.22047 95.374) (end 153.34647 93.5) (width 0.25) (layer "F.Cu") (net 13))
 (segment (start 73.674 67.373562) (end 74.216438 67.916) (width 0.25) (layer "F.Cu") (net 13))
 (segment (start 74.25 66.064) (end 74.216438 66.064) (width 0.25) (layer "F.Cu") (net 13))
 (segment (start 74.25 65.376) (end 74.25 66.064) (width 0.25) (layer "F.Cu") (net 13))
 (segment (start 150.25 93.5) (end 112.649 55.899) (width 0.25) (layer "F.Cu") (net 13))
 (segment (start 75.783562 68.604) (end 76.326 69.146438) (width 0.25) (layer "F.Cu") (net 13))
 (segment (start 74.25 67.916) (end 74.25 68.14219) (width 0.25) (layer "F.Cu") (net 13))
 (segment (start 164.75 92.25) (end 161.626 95.374) (width 0.25) (layer "F.Cu") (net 13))
 (segment (start 76.326 69.913562) (end 75.783562 70.456) (width 0.25) (layer "F.Cu") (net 13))
 (segment (start 76.101 55.899) (end 74.25 57.75) (width 0.25) (layer "F.Cu") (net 13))
 (segment (start 74.71181 68.604) (end 75.783562 68.604) (width 0.25) (layer "F.Cu") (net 13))
 (segment (start 74.25 70.717546) (end 75.301227 71.768773) (width 0.25) (layer "F.Cu") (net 13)))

